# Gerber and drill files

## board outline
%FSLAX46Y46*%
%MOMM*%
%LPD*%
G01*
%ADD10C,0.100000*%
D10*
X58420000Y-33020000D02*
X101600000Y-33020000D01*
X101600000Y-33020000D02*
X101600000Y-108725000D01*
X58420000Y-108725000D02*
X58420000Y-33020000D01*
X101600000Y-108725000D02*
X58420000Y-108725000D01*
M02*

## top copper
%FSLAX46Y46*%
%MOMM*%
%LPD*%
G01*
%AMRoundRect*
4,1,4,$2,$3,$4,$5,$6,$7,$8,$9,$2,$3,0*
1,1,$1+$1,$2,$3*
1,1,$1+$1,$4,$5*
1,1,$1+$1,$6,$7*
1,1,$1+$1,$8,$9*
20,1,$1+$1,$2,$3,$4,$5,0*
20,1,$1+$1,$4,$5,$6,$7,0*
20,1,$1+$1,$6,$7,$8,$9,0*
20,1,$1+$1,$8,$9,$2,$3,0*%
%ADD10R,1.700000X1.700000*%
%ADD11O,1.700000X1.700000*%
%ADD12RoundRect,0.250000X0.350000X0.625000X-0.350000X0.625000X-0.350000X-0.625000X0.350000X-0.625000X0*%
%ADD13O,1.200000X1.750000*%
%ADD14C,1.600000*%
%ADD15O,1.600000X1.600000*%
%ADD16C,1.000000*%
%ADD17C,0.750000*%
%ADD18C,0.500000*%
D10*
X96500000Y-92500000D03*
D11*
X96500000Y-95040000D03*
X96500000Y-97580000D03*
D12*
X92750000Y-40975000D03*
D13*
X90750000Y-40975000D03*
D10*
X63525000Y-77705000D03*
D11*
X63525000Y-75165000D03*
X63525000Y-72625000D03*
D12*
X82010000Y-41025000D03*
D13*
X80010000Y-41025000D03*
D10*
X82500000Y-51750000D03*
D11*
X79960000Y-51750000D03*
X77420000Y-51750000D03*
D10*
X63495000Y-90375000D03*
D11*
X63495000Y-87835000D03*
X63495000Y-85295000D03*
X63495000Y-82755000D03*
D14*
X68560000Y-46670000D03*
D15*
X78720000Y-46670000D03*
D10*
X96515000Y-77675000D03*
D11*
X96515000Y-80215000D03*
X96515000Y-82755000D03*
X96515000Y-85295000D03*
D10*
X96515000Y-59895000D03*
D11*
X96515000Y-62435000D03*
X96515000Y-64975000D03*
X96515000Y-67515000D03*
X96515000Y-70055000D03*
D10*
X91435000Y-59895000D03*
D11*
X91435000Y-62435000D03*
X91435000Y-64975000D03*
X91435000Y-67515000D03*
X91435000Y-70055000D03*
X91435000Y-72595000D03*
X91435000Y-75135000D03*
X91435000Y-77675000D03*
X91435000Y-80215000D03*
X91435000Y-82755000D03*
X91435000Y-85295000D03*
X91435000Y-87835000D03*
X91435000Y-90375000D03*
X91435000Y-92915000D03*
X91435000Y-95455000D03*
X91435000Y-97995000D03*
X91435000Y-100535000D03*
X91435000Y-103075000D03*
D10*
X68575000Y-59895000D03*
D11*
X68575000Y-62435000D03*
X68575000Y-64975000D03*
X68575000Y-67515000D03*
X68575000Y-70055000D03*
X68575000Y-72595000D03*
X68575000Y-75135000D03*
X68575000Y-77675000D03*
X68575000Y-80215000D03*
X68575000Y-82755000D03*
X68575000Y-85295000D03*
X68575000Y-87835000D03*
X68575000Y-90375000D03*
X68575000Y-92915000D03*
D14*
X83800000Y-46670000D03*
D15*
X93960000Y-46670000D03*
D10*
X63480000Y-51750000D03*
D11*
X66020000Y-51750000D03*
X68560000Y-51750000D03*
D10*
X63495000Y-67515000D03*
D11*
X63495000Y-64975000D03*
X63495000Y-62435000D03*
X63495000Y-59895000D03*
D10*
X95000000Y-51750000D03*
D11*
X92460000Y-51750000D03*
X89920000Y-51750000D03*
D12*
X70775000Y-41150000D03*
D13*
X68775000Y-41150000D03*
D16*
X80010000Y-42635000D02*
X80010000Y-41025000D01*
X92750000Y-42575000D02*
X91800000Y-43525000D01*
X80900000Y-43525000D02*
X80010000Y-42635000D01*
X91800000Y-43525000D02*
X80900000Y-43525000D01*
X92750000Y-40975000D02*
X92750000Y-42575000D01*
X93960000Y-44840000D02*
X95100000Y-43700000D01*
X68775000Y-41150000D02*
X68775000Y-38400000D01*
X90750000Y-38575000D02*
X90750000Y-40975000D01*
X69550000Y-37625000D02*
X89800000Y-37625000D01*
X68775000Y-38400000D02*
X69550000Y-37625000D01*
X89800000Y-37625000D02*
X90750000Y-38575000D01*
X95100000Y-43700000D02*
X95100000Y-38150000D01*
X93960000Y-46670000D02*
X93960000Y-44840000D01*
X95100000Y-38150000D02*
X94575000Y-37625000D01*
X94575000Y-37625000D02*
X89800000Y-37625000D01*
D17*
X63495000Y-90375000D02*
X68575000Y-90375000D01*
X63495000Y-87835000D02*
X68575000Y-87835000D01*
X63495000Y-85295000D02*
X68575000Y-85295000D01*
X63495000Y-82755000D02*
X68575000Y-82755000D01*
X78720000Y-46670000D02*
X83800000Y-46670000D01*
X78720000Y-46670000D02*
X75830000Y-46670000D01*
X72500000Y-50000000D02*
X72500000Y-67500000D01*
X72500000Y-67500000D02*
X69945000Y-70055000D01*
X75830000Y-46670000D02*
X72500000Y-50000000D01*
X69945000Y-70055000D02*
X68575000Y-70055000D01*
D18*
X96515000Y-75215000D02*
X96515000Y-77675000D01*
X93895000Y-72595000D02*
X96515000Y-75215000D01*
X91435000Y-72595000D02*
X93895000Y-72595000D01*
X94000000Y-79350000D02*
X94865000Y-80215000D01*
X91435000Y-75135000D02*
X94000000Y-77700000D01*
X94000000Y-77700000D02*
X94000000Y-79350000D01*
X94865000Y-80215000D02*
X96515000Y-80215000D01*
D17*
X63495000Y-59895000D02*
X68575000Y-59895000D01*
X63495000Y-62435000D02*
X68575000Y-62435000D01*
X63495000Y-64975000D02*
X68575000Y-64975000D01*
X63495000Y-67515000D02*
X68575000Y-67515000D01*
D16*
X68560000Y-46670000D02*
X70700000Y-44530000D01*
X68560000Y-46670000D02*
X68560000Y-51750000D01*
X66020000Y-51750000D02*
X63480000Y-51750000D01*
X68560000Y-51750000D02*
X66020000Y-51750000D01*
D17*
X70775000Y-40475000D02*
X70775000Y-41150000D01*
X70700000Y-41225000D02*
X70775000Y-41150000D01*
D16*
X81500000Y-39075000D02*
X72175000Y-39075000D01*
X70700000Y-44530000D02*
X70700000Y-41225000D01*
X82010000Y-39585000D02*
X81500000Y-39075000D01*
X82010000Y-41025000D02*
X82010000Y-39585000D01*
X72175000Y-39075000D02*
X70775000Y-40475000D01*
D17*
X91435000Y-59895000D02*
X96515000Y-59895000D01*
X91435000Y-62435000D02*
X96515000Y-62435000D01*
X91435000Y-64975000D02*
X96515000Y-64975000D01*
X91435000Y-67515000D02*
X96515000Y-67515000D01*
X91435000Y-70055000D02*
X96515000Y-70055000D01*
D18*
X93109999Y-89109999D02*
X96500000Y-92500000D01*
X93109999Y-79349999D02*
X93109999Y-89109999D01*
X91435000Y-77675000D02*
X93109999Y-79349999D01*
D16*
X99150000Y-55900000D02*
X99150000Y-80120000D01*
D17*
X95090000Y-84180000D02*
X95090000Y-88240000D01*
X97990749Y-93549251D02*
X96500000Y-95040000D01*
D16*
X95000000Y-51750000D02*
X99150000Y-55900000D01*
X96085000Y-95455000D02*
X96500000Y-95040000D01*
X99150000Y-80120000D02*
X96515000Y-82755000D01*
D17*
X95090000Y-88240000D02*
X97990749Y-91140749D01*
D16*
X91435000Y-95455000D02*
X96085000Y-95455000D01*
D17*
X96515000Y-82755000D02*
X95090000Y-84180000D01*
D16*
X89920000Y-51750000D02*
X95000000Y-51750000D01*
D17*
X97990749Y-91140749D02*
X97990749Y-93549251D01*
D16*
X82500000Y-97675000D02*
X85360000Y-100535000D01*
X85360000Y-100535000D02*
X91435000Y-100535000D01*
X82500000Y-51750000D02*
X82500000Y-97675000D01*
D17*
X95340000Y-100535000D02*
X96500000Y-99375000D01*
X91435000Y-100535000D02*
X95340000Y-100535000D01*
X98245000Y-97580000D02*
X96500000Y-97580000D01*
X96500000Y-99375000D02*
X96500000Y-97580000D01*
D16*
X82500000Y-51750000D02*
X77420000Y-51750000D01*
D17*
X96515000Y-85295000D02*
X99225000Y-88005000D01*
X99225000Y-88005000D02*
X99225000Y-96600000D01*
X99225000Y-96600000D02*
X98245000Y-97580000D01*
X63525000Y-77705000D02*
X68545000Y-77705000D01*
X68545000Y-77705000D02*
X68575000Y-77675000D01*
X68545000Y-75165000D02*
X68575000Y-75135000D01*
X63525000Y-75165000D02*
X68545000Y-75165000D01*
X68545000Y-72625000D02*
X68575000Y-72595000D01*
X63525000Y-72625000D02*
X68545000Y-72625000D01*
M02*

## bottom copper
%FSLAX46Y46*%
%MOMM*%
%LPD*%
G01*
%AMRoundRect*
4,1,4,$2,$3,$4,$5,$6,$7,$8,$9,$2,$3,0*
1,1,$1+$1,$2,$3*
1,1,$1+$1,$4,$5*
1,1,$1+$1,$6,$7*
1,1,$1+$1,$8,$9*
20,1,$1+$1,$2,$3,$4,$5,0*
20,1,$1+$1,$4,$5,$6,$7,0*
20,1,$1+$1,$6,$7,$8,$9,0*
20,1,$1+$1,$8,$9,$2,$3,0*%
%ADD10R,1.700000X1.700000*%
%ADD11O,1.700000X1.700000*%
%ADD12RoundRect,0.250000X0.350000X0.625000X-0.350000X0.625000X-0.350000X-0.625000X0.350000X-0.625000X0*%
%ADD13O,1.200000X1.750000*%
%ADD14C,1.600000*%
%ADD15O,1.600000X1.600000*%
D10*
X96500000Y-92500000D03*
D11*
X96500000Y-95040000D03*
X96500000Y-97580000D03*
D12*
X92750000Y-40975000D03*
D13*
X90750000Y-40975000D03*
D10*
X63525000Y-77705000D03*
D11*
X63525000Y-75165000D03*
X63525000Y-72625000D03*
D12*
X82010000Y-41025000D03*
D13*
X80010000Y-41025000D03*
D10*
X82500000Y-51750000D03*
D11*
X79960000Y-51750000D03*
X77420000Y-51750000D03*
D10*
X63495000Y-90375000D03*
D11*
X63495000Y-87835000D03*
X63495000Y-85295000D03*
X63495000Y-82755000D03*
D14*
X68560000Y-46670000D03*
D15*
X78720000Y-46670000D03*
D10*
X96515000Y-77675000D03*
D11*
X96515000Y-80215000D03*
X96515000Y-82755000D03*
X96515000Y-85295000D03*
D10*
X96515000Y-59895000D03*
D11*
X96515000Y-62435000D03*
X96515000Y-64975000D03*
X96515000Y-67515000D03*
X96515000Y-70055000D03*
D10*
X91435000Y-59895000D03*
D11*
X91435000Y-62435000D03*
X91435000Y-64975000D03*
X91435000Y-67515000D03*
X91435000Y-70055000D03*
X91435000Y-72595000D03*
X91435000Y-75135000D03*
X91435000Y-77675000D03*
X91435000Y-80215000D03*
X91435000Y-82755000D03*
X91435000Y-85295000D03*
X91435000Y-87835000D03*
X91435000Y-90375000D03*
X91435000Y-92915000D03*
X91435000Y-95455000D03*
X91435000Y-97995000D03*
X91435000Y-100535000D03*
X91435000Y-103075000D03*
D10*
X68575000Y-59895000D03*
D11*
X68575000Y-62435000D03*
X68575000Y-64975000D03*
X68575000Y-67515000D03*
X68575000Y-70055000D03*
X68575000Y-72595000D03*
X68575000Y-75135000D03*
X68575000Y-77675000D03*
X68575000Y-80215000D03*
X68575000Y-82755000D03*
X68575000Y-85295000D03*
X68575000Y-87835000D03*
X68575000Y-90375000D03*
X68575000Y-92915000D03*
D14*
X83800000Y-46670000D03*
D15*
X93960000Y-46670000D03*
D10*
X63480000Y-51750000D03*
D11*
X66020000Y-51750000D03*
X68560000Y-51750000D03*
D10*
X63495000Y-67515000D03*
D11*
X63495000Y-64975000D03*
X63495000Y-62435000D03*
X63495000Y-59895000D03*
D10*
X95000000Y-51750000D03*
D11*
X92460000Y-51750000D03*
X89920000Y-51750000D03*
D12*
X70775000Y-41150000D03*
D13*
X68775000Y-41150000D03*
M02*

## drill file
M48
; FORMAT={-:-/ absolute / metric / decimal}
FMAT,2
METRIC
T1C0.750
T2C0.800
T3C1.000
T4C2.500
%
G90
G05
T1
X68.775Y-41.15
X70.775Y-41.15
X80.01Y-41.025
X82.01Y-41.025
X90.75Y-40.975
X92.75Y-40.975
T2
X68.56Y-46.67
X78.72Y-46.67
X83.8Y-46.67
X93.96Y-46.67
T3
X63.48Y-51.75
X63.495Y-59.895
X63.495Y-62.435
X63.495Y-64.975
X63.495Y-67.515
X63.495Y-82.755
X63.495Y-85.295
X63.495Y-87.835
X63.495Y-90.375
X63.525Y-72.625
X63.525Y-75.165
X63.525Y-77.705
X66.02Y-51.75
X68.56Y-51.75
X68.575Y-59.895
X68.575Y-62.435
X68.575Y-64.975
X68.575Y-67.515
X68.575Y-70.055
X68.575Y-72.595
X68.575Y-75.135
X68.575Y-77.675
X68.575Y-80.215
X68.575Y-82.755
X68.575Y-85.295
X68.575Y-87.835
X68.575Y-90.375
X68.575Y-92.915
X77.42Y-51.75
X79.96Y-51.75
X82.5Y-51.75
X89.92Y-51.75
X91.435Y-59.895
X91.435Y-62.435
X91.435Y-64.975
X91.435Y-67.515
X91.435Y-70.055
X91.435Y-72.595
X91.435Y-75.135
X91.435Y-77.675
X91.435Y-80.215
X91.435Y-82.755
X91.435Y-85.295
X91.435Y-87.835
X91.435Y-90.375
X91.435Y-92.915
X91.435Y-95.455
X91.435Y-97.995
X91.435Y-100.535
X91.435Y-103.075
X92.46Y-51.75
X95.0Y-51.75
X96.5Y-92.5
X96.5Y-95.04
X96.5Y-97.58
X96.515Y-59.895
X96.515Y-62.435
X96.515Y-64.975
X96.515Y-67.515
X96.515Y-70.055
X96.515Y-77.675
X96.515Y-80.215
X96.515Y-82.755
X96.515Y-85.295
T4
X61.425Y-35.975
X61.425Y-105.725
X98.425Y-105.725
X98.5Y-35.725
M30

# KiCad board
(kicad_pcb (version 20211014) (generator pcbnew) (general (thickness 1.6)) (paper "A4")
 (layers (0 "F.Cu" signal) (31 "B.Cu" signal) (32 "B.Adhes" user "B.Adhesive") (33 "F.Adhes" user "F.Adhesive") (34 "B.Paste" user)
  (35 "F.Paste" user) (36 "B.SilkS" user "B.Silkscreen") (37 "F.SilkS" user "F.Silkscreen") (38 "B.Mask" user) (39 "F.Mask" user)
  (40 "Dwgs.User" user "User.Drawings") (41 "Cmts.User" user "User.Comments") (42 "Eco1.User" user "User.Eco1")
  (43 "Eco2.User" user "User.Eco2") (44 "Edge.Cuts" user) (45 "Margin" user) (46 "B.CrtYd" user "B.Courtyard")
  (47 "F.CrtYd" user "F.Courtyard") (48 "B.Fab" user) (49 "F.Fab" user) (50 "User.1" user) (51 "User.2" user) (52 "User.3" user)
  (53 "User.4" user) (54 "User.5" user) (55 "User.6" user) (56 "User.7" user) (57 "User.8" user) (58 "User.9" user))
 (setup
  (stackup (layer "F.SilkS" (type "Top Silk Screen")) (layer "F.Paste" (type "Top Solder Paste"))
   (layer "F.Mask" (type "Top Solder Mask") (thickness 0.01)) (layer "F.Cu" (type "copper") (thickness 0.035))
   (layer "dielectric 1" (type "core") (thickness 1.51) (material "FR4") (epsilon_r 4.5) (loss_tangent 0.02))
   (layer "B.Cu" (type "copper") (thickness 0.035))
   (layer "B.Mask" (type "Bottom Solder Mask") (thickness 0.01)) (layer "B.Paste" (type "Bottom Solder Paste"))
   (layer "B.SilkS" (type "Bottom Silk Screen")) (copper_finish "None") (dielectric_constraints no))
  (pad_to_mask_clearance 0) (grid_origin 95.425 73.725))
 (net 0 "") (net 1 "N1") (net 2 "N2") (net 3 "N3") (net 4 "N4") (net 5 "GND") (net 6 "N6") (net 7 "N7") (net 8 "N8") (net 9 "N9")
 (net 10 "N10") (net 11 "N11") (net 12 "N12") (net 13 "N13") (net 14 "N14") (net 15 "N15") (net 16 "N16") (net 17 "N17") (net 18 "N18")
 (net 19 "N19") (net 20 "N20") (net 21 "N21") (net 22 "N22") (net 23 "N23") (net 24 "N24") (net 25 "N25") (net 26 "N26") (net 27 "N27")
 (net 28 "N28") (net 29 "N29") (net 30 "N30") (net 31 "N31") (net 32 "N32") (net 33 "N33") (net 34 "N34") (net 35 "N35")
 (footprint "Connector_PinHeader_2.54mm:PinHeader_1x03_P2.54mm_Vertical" (layer "F.Cu") (at 96.5 92.5)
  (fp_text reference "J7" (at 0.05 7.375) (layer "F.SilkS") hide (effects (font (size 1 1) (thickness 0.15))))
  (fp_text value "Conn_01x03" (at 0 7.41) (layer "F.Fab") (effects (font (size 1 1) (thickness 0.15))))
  (pad "1" thru_hole rect (at 0 0) (size 1.7 1.7) (drill 1) (layers *.Cu *.Mask) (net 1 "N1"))
  (pad "2" thru_hole oval (at 0 2.54) (size 1.7 1.7) (drill 1) (layers *.Cu *.Mask) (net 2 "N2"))
  (pad "3" thru_hole oval (at 0 5.08) (size 1.7 1.7) (drill 1) (layers *.Cu *.Mask) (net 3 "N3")))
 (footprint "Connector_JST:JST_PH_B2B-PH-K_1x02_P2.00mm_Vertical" (layer "F.Cu") (at 92.75 40.975 180)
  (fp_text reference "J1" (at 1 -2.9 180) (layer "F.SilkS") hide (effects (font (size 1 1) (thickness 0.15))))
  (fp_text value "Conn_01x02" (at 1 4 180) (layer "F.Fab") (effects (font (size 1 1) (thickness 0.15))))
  (pad "1" thru_hole roundrect (at 0 0 180) (size 1.2 1.75) (drill 0.75) (layers *.Cu *.Mask) (roundrect_rratio 0.2083333333) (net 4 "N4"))
  (pad "2" thru_hole oval (at 2 0 180) (size 1.2 1.75) (drill 0.75) (layers *.Cu *.Mask) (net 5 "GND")))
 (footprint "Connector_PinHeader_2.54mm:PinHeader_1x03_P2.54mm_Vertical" (layer "F.Cu") (at 63.525 77.705 180)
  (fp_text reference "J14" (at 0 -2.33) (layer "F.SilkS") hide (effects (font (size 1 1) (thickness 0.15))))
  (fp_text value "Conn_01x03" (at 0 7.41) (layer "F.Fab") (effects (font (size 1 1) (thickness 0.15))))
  (pad "1" thru_hole rect (at 0 0 180) (size 1.7 1.7) (drill 1) (layers *.Cu *.Mask) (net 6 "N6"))
  (pad "2" thru_hole oval (at 0 2.54 180) (size 1.7 1.7) (drill 1) (layers *.Cu *.Mask) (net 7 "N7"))
  (pad "3" thru_hole oval (at 0 5.08 180) (size 1.7 1.7) (drill 1) (layers *.Cu *.Mask) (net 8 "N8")))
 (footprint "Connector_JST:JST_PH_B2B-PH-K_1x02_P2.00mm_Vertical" (layer "F.Cu") (at 82.01 41.025 180)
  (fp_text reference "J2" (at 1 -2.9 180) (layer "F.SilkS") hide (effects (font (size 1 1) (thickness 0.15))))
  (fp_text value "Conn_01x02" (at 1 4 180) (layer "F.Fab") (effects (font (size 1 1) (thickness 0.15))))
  (pad "1" thru_hole roundrect (at 0 0 180) (size 1.2 1.75) (drill 0.75) (layers *.Cu *.Mask) (roundrect_rratio 0.2083333333) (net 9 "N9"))
  (pad "2" thru_hole oval (at 2 0 180) (size 1.2 1.75) (drill 0.75) (layers *.Cu *.Mask) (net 4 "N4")))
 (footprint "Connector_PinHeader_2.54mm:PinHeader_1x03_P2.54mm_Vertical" (layer "F.Cu") (at 82.5 51.75 -90)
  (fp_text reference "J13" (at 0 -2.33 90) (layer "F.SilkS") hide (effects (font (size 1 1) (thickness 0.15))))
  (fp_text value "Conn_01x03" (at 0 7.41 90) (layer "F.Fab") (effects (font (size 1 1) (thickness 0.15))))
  (pad "1" thru_hole rect (at 0 0 270) (size 1.7 1.7) (drill 1) (layers *.Cu *.Mask) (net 3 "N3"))
  (pad "2" thru_hole oval (at 0 2.54 270) (size 1.7 1.7) (drill 1) (layers *.Cu *.Mask) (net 3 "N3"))
  (pad "3" thru_hole oval (at 0 5.08 270) (size 1.7 1.7) (drill 1) (layers *.Cu *.Mask) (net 3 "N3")))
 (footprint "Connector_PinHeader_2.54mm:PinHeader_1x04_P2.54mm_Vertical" (layer "F.Cu") (at 63.495 90.375 180)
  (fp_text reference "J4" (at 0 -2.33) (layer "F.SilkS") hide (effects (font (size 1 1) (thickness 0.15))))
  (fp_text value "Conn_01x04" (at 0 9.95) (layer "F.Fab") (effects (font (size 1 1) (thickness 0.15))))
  (pad "1" thru_hole rect (at 0 0 180) (size 1.7 1.7) (drill 1) (layers *.Cu *.Mask) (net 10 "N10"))
  (pad "2" thru_hole oval (at 0 2.54 180) (size 1.7 1.7) (drill 1) (layers *.Cu *.Mask) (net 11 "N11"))
  (pad "3" thru_hole oval (at 0 5.08 180) (size 1.7 1.7) (drill 1) (layers *.Cu *.Mask) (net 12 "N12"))
  (pad "4" thru_hole oval (at 0 7.62 180) (size 1.7 1.7) (drill 1) (layers *.Cu *.Mask) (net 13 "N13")))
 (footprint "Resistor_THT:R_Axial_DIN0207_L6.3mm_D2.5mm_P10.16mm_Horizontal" (layer "F.Cu") (at 68.56 46.67)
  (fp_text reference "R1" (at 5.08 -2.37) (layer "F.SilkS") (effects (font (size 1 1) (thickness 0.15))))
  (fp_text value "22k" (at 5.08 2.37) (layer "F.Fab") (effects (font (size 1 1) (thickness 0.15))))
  (pad "1" thru_hole circle (at 0 0) (size 1.6 1.6) (drill 0.8) (layers *.Cu *.Mask) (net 9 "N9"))
  (pad "2" thru_hole oval (at 10.16 0) (size 1.6 1.6) (drill 0.8) (layers *.Cu *.Mask) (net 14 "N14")))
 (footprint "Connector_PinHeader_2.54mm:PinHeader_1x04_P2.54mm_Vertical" (layer "F.Cu") (at 96.515 77.675)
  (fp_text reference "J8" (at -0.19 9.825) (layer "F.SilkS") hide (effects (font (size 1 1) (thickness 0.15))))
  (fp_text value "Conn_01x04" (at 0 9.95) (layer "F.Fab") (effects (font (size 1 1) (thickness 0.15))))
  (pad "1" thru_hole rect (at 0 0) (size 1.7 1.7) (drill 1) (layers *.Cu *.Mask) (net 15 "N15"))
  (pad "2" thru_hole oval (at 0 2.54) (size 1.7 1.7) (drill 1) (layers *.Cu *.Mask) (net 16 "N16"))
  (pad "3" thru_hole oval (at 0 5.08) (size 1.7 1.7) (drill 1) (layers *.Cu *.Mask) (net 2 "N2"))
  (pad "4" thru_hole oval (at 0 7.62) (size 1.7 1.7) (drill 1) (layers *.Cu *.Mask) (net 3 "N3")))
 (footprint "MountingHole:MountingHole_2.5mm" (layer "F.Cu") (at 98.425 35.725)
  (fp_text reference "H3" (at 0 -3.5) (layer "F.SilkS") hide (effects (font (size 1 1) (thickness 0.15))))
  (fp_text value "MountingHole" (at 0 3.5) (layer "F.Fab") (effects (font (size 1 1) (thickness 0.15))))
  (pad "" np_thru_hole circle (at 0.075 0) (size 2.5 2.5) (drill 2.5) (layers F&B.Cu *.Mask)))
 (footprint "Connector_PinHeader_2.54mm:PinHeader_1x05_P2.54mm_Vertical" (layer "F.Cu") (at 96.515 59.895)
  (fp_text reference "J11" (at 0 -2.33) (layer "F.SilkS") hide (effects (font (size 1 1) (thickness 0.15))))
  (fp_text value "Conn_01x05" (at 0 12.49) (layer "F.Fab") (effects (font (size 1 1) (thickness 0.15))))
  (pad "1" thru_hole rect (at 0 0) (size 1.7 1.7) (drill 1) (layers *.Cu *.Mask) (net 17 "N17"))
  (pad "2" thru_hole oval (at 0 2.54) (size 1.7 1.7) (drill 1) (layers *.Cu *.Mask) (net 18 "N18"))
  (pad "3" thru_hole oval (at 0 5.08) (size 1.7 1.7) (drill 1) (layers *.Cu *.Mask) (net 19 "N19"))
  (pad "4" thru_hole oval (at 0 7.62) (size 1.7 1.7) (drill 1) (layers *.Cu *.Mask) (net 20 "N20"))
  (pad "5" thru_hole oval (at 0 10.16) (size 1.7 1.7) (drill 1) (layers *.Cu *.Mask) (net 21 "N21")))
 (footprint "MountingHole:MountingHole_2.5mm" (layer "F.Cu") (at 61.425 35.975)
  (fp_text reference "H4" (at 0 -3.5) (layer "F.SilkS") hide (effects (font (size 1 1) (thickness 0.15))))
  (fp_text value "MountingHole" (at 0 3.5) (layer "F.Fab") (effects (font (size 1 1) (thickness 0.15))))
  (pad "" np_thru_hole circle (at 0 0) (size 2.5 2.5) (drill 2.5) (layers *.Cu *.Mask)))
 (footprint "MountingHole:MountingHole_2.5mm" (layer "F.Cu") (at 98.425 105.725)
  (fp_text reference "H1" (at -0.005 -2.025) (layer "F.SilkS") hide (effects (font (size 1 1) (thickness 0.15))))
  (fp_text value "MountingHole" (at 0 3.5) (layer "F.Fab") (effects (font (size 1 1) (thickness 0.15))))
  (pad "" np_thru_hole circle (at 0 0) (size 2.5 2.5) (drill 2.5) (layers *.Cu *.Mask)))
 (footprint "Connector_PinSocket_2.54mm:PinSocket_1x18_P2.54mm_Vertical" (layer "F.Cu") (at 91.435 59.895)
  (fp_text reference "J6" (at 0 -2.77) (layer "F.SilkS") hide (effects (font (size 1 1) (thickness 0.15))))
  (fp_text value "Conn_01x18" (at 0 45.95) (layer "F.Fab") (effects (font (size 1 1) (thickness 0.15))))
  (pad "1" thru_hole rect (at 0 0) (size 1.7 1.7) (drill 1) (layers *.Cu *.Mask) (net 17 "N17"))
  (pad "2" thru_hole oval (at 0 2.54) (size 1.7 1.7) (drill 1) (layers *.Cu *.Mask) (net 18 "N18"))
  (pad "3" thru_hole oval (at 0 5.08) (size 1.7 1.7) (drill 1) (layers *.Cu *.Mask) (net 19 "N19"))
  (pad "4" thru_hole oval (at 0 7.62) (size 1.7 1.7) (drill 1) (layers *.Cu *.Mask) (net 20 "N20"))
  (pad "5" thru_hole oval (at 0 10.16) (size 1.7 1.7) (drill 1) (layers *.Cu *.Mask) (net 21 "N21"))
  (pad "6" thru_hole oval (at 0 12.7) (size 1.7 1.7) (drill 1) (layers *.Cu *.Mask) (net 15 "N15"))
  (pad "7" thru_hole oval (at 0 15.24) (size 1.7 1.7) (drill 1) (layers *.Cu *.Mask) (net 16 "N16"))
  (pad "8" thru_hole oval (at 0 17.78) (size 1.7 1.7) (drill 1) (layers *.Cu *.Mask) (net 1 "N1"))
  (pad "9" thru_hole oval (at 0 20.32) (size 1.7 1.7) (drill 1) (layers *.Cu *.Mask) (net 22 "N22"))
  (pad "10" thru_hole oval (at 0 22.86) (size 1.7 1.7) (drill 1) (layers *.Cu *.Mask) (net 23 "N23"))
  (pad "11" thru_hole oval (at 0 25.4) (size 1.7 1.7) (drill 1) (layers *.Cu *.Mask) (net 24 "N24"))
  (pad "12" thru_hole oval (at 0 27.94) (size 1.7 1.7) (drill 1) (layers *.Cu *.Mask) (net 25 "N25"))
  (pad "13" thru_hole oval (at 0 30.48) (size 1.7 1.7) (drill 1) (layers *.Cu *.Mask) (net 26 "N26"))
  (pad "14" thru_hole oval (at 0 33.02) (size 1.7 1.7) (drill 1) (layers *.Cu *.Mask) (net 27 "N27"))
  (pad "15" thru_hole oval (at 0 35.56) (size 1.7 1.7) (drill 1) (layers *.Cu *.Mask) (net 2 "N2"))
  (pad "16" thru_hole oval (at 0 38.1) (size 1.7 1.7) (drill 1) (layers *.Cu *.Mask) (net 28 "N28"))
  (pad "17" thru_hole oval (at 0 40.64) (size 1.7 1.7) (drill 1) (layers *.Cu *.Mask) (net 3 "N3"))
  (pad "18" thru_hole oval (at 0 43.18) (size 1.7 1.7) (drill 1) (layers *.Cu *.Mask) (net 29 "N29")))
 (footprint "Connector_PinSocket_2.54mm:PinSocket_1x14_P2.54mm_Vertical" (layer "F.Cu") (at 68.575 59.895)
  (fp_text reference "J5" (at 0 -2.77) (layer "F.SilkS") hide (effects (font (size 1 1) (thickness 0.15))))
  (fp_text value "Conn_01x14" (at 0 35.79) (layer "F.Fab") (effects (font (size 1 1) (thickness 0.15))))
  (pad "1" thru_hole rect (at 0 0) (size 1.7 1.7) (drill 1) (layers *.Cu *.Mask) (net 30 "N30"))
  (pad "2" thru_hole oval (at 0 2.54) (size 1.7 1.7) (drill 1) (layers *.Cu *.Mask) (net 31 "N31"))
  (pad "3" thru_hole oval (at 0 5.08) (size 1.7 1.7) (drill 1) (layers *.Cu *.Mask) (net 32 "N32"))
  (pad "4" thru_hole oval (at 0 7.62) (size 1.7 1.7) (drill 1) (layers *.Cu *.Mask) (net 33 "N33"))
  (pad "5" thru_hole oval (at 0 10.16) (size 1.7 1.7) (drill 1) (layers *.Cu *.Mask) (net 14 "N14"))
  (pad "6" thru_hole oval (at 0 12.7) (size 1.7 1.7) (drill 1) (layers *.Cu *.Mask) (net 8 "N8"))
  (pad "7" thru_hole oval (at 0 15.24) (size 1.7 1.7) (drill 1) (layers *.Cu *.Mask) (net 7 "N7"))
  (pad "8" thru_hole oval (at 0 17.78) (size 1.7 1.7) (drill 1) (layers *.Cu *.Mask) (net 6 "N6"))
  (pad "9" thru_hole oval (at 0 20.32) (size 1.7 1.7) (drill 1) (layers *.Cu *.Mask) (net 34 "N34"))
  (pad "10" thru_hole oval (at 0 22.86) (size 1.7 1.7) (drill 1) (layers *.Cu *.Mask) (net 13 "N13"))
  (pad "11" thru_hole oval (at 0 25.4) (size 1.7 1.7) (drill 1) (layers *.Cu *.Mask) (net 12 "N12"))
  (pad "12" thru_hole oval (at 0 27.94) (size 1.7 1.7) (drill 1) (layers *.Cu *.Mask) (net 11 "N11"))
  (pad "13" thru_hole oval (at 0 30.48) (size 1.7 1.7) (drill 1) (layers *.Cu *.Mask) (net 10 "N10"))
  (pad "14" thru_hole oval (at 0 33.02) (size 1.7 1.7) (drill 1) (layers *.Cu *.Mask) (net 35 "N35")))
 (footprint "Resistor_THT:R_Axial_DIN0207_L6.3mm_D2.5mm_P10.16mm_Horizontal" (layer "F.Cu") (at 83.8 46.67)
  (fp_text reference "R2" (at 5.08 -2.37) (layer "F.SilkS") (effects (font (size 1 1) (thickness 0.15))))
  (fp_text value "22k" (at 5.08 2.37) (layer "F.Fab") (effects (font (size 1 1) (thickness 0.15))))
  (pad "1" thru_hole circle (at 0 0) (size 1.6 1.6) (drill 0.8) (layers *.Cu *.Mask) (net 14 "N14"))
  (pad "2" thru_hole oval (at 10.16 0) (size 1.6 1.6) (drill 0.8) (layers *.Cu *.Mask) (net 5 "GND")))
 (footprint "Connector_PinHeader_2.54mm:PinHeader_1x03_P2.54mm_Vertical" (layer "F.Cu") (at 63.48 51.75 90)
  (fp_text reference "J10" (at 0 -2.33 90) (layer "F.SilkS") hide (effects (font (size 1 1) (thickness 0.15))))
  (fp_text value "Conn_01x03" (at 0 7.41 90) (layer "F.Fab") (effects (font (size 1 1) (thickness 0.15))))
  (pad "1" thru_hole rect (at 0 0 90) (size 1.7 1.7) (drill 1) (layers *.Cu *.Mask) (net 9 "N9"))
  (pad "2" thru_hole oval (at 0 2.54 90) (size 1.7 1.7) (drill 1) (layers *.Cu *.Mask) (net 9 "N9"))
  (pad "3" thru_hole oval (at 0 5.08 90) (size 1.7 1.7) (drill 1) (layers *.Cu *.Mask) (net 9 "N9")))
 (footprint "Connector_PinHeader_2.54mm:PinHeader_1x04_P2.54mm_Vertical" (layer "F.Cu") (at 63.495 67.515 180)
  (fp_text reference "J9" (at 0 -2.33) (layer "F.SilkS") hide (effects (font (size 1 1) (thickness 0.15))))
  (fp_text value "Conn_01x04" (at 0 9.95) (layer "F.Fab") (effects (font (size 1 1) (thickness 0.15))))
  (pad "1" thru_hole rect (at 0 0 180) (size 1.7 1.7) (drill 1) (layers *.Cu *.Mask) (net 33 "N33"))
  (pad "2" thru_hole oval (at 0 2.54 180) (size 1.7 1.7) (drill 1) (layers *.Cu *.Mask) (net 32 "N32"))
  (pad "3" thru_hole oval (at 0 5.08 180) (size 1.7 1.7) (drill 1) (layers *.Cu *.Mask) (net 31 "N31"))
  (pad "4" thru_hole oval (at 0 7.62 180) (size 1.7 1.7) (drill 1) (layers *.Cu *.Mask) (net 30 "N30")))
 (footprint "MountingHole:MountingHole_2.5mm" (layer "F.Cu") (at 61.425 105.725)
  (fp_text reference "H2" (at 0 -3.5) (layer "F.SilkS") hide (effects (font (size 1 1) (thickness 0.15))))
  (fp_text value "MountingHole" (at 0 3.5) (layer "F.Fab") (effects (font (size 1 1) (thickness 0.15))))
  (pad "" np_thru_hole circle (at 0 0) (size 2.5 2.5) (drill 2.5) (layers *.Cu *.Mask)))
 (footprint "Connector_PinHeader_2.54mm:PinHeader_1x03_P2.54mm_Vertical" (layer "F.Cu") (at 95 51.75 -90)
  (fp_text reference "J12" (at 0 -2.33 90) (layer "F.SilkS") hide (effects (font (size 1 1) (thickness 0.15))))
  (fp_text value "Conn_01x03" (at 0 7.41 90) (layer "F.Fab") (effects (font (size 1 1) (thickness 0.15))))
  (pad "1" thru_hole rect (at 0 0 270) (size 1.7 1.7) (drill 1) (layers *.Cu *.Mask) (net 2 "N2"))
  (pad "2" thru_hole oval (at 0 2.54 270) (size 1.7 1.7) (drill 1) (layers *.Cu *.Mask) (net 2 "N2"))
  (pad "3" thru_hole oval (at 0 5.08 270) (size 1.7 1.7) (drill 1) (layers *.Cu *.Mask) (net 2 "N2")))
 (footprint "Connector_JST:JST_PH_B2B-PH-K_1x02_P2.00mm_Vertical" (layer "F.Cu") (at 70.775 41.15 180)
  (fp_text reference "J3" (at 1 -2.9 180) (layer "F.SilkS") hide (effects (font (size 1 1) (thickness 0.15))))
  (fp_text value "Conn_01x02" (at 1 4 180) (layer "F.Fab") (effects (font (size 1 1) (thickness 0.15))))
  (pad "1" thru_hole roundrect (at 0 0 180) (size 1.2 1.75) (drill 0.75) (layers *.Cu *.Mask) (roundrect_rratio 0.2083333333) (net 9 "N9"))
  (pad "2" thru_hole oval (at 2 0 180) (size 1.2 1.75) (drill 0.75) (layers *.Cu *.Mask) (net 5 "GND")))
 (gr_line (start 58.42 33.02) (end 101.6 33.02) (layer "Edge.Cuts") (width 0.1))
 (gr_line (start 101.6 33.02) (end 101.6 108.725) (layer "Edge.Cuts") (width 0.1))
 (gr_line (start 58.42 108.725) (end 58.42 33.02) (layer "Edge.Cuts") (width 0.1))
 (gr_line (start 101.6 108.725) (end 58.42 108.725) (layer "Edge.Cuts") (width 0.1))
 (segment (start 80.01 42.635) (end 80.01 41.025) (width 1) (layer "F.Cu") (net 4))
 (segment (start 92.75 42.575) (end 91.8 43.525) (width 1) (layer "F.Cu") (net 4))
 (segment (start 80.9 43.525) (end 80.01 42.635) (width 1) (layer "F.Cu") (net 4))
 (segment (start 91.8 43.525) (end 80.9 43.525) (width 1) (layer "F.Cu") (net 4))
 (segment (start 92.75 40.975) (end 92.75 42.575) (width 1) (layer "F.Cu") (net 4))
 (segment (start 93.96 44.84) (end 95.1 43.7) (width 1) (layer "F.Cu") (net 5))
 (segment (start 68.775 41.15) (end 68.775 38.4) (width 1) (layer "F.Cu") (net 5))
 (segment (start 90.75 38.575) (end 90.75 40.975) (width 1) (layer "F.Cu") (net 5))
 (segment (start 69.55 37.625) (end 89.8 37.625) (width 1) (layer "F.Cu") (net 5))
 (segment (start 68.775 38.4) (end 69.55 37.625) (width 1) (layer "F.Cu") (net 5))
 (segment (start 89.8 37.625) (end 90.75 38.575) (width 1) (layer "F.Cu") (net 5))
 (segment (start 95.1 43.7) (end 95.1 38.15) (width 1) (layer "F.Cu") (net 5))
 (segment (start 93.96 46.67) (end 93.96 44.84) (width 1) (layer "F.Cu") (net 5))
 (segment (start 95.1 38.15) (end 94.575 37.625) (width 1) (layer "F.Cu") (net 5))
 (segment (start 94.575 37.625) (end 89.8 37.625) (width 1) (layer "F.Cu") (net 5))
 (segment (start 63.495 90.375) (end 68.575 90.375) (width 0.75) (layer "F.Cu") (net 10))
 (segment (start 63.495 87.835) (end 68.575 87.835) (width 0.75) (layer "F.Cu") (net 11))
 (segment (start 63.495 85.295) (end 68.575 85.295) (width 0.75) (layer "F.Cu") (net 12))
 (segment (start 63.495 82.755) (end 68.575 82.755) (width 0.75) (layer "F.Cu") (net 13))
 (segment (start 78.72 46.67) (end 83.8 46.67) (width 0.75) (layer "F.Cu") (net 14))
 (segment (start 78.72 46.67) (end 75.83 46.67) (width 0.75) (layer "F.Cu") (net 14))
 (segment (start 72.5 50) (end 72.5 67.5) (width 0.75) (layer "F.Cu") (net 14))
 (segment (start 72.5 67.5) (end 69.945 70.055) (width 0.75) (layer "F.Cu") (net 14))
 (segment (start 75.83 46.67) (end 72.5 50) (width 0.75) (layer "F.Cu") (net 14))
 (segment (start 69.945 70.055) (end 68.575 70.055) (width 0.75) (layer "F.Cu") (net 14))
 (segment (start 96.515 75.215) (end 96.515 77.675) (width 0.5) (layer "F.Cu") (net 15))
 (segment (start 93.895 72.595) (end 96.515 75.215) (width 0.5) (layer "F.Cu") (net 15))
 (segment (start 91.435 72.595) (end 93.895 72.595) (width 0.5) (layer "F.Cu") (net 15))
 (segment (start 94 79.35) (end 94.865 80.215) (width 0.5) (layer "F.Cu") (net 16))
 (segment (start 91.435 75.135) (end 94 77.7) (width 0.5) (layer "F.Cu") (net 16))
 (segment (start 94 77.7) (end 94 79.35) (width 0.5) (layer "F.Cu") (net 16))
 (segment (start 94.865 80.215) (end 96.515 80.215) (width 0.5) (layer "F.Cu") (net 16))
 (segment (start 63.495 59.895) (end 68.575 59.895) (width 0.75) (layer "F.Cu") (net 30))
 (segment (start 63.495 62.435) (end 68.575 62.435) (width 0.75) (layer "F.Cu") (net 31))
 (segment (start 63.495 64.975) (end 68.575 64.975) (width 0.75) (layer "F.Cu") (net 32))
 (segment (start 63.495 67.515) (end 68.575 67.515) (width 0.75) (layer "F.Cu") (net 33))
 (segment (start 68.56 46.67) (end 70.7 44.53) (width 1) (layer "F.Cu") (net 9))
 (segment (start 68.56 46.67) (end 68.56 51.75) (width 1) (layer "F.Cu") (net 9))
 (segment (start 66.02 51.75) (end 63.48 51.75) (width 1) (layer "F.Cu") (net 9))
 (segment (start 68.56 51.75) (end 66.02 51.75) (width 1) (layer "F.Cu") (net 9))
 (segment (start 70.775 40.475) (end 70.775 41.15) (width 0.75) (layer "F.Cu") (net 9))
 (segment (start 70.7 41.225) (end 70.775 41.15) (width 0.75) (layer "F.Cu") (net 9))
 (segment (start 81.5 39.075) (end 72.175 39.075) (width 1) (layer "F.Cu") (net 9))
 (segment (start 70.7 44.53) (end 70.7 41.225) (width 1) (layer "F.Cu") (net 9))
 (segment (start 82.01 39.585) (end 81.5 39.075) (width 1) (layer "F.Cu") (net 9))
 (segment (start 82.01 41.025) (end 82.01 39.585) (width 1) (layer "F.Cu") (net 9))
 (segment (start 72.175 39.075) (end 70.775 40.475) (width 1) (layer "F.Cu") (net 9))
 (segment (start 91.435 59.895) (end 96.515 59.895) (width 0.75) (layer "F.Cu") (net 17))
 (segment (start 91.435 62.435) (end 96.515 62.435) (width 0.75) (layer "F.Cu") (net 18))
 (segment (start 91.435 64.975) (end 96.515 64.975) (width 0.75) (layer "F.Cu") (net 19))
 (segment (start 91.435 67.515) (end 96.515 67.515) (width 0.75) (layer "F.Cu") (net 20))
 (segment (start 91.435 70.055) (end 96.515 70.055) (width 0.75) (layer "F.Cu") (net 21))
 (segment (start 93.109999 89.109999) (end 96.5 92.5) (width 0.5) (layer "F.Cu") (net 1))
 (segment (start 93.109999 79.349999) (end 93.109999 89.109999) (width 0.5) (layer "F.Cu") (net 1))
 (segment (start 91.435 77.675) (end 93.109999 79.349999) (width 0.5) (layer "F.Cu") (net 1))
 (segment (start 99.15 55.9) (end 99.15 80.12) (width 1) (layer "F.Cu") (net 2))
 (segment (start 95.09 84.18) (end 95.09 88.24) (width 0.75) (layer "F.Cu") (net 2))
 (segment (start 97.990749 93.549251) (end 96.5 95.04) (width 0.75) (layer "F.Cu") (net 2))
 (segment (start 95 51.75) (end 99.15 55.9) (width 1) (layer "F.Cu") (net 2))
 (segment (start 96.085 95.455) (end 96.5 95.04) (width 1) (layer "F.Cu") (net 2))
 (segment (start 99.15 80.12) (end 96.515 82.755) (width 1) (layer "F.Cu") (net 2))
 (segment (start 95.09 88.24) (end 97.990749 91.140749) (width 0.75) (layer "F.Cu") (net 2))
 (segment (start 91.435 95.455) (end 96.085 95.455) (width 1) (layer "F.Cu") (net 2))
 (segment (start 96.515 82.755) (end 95.09 84.18) (width 0.75) (layer "F.Cu") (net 2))
 (segment (start 89.92 51.75) (end 95 51.75) (width 1) (layer "F.Cu") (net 2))
 (segment (start 97.990749 91.140749) (end 97.990749 93.549251) (width 0.75) (layer "F.Cu") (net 2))
 (segment (start 82.5 97.675) (end 85.36 100.535) (width 1) (layer "F.Cu") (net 3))
 (segment (start 85.36 100.535) (end 91.435 100.535) (width 1) (layer "F.Cu") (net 3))
 (segment (start 82.5 51.75) (end 82.5 97.675) (width 1) (layer "F.Cu") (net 3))
 (segment (start 95.34 100.535) (end 96.5 99.375) (width 0.75) (layer "F.Cu") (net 3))
 (segment (start 91.435 100.535) (end 95.34 100.535) (width 0.75) (layer "F.Cu") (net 3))
 (segment (start 98.245 97.58) (end 96.5 97.58) (width 0.75) (layer "F.Cu") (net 3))
 (segment (start 96.5 99.375) (end 96.5 97.58) (width 0.75) (layer "F.Cu") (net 3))
 (segment (start 82.5 51.75) (end 77.42 51.75) (width 1) (layer "F.Cu") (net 3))
 (segment (start 96.515 85.295) (end 99.225 88.005) (width 0.75) (layer "F.Cu") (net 3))
 (segment (start 99.225 88.005) (end 99.225 96.6) (width 0.75) (layer "F.Cu") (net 3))
 (segment (start 99.225 96.6) (end 98.245 97.58) (width 0.75) (layer "F.Cu") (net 3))
 (segment (start 63.525 77.705) (end 68.545 77.705) (width 0.75) (layer "F.Cu") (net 6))
 (segment (start 68.545 77.705) (end 68.575 77.675) (width 0.75) (layer "F.Cu") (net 6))
 (segment (start 68.545 75.165) (end 68.575 75.135) (width 0.75) (layer "F.Cu") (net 7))
 (segment (start 63.525 75.165) (end 68.545 75.165) (width 0.75) (layer "F.Cu") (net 7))
 (segment (start 68.545 72.625) (end 68.575 72.595) (width 0.75) (layer "F.Cu") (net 8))
 (segment (start 63.525 72.625) (end 68.545 72.625) (width 0.75) (layer "F.Cu") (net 8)))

